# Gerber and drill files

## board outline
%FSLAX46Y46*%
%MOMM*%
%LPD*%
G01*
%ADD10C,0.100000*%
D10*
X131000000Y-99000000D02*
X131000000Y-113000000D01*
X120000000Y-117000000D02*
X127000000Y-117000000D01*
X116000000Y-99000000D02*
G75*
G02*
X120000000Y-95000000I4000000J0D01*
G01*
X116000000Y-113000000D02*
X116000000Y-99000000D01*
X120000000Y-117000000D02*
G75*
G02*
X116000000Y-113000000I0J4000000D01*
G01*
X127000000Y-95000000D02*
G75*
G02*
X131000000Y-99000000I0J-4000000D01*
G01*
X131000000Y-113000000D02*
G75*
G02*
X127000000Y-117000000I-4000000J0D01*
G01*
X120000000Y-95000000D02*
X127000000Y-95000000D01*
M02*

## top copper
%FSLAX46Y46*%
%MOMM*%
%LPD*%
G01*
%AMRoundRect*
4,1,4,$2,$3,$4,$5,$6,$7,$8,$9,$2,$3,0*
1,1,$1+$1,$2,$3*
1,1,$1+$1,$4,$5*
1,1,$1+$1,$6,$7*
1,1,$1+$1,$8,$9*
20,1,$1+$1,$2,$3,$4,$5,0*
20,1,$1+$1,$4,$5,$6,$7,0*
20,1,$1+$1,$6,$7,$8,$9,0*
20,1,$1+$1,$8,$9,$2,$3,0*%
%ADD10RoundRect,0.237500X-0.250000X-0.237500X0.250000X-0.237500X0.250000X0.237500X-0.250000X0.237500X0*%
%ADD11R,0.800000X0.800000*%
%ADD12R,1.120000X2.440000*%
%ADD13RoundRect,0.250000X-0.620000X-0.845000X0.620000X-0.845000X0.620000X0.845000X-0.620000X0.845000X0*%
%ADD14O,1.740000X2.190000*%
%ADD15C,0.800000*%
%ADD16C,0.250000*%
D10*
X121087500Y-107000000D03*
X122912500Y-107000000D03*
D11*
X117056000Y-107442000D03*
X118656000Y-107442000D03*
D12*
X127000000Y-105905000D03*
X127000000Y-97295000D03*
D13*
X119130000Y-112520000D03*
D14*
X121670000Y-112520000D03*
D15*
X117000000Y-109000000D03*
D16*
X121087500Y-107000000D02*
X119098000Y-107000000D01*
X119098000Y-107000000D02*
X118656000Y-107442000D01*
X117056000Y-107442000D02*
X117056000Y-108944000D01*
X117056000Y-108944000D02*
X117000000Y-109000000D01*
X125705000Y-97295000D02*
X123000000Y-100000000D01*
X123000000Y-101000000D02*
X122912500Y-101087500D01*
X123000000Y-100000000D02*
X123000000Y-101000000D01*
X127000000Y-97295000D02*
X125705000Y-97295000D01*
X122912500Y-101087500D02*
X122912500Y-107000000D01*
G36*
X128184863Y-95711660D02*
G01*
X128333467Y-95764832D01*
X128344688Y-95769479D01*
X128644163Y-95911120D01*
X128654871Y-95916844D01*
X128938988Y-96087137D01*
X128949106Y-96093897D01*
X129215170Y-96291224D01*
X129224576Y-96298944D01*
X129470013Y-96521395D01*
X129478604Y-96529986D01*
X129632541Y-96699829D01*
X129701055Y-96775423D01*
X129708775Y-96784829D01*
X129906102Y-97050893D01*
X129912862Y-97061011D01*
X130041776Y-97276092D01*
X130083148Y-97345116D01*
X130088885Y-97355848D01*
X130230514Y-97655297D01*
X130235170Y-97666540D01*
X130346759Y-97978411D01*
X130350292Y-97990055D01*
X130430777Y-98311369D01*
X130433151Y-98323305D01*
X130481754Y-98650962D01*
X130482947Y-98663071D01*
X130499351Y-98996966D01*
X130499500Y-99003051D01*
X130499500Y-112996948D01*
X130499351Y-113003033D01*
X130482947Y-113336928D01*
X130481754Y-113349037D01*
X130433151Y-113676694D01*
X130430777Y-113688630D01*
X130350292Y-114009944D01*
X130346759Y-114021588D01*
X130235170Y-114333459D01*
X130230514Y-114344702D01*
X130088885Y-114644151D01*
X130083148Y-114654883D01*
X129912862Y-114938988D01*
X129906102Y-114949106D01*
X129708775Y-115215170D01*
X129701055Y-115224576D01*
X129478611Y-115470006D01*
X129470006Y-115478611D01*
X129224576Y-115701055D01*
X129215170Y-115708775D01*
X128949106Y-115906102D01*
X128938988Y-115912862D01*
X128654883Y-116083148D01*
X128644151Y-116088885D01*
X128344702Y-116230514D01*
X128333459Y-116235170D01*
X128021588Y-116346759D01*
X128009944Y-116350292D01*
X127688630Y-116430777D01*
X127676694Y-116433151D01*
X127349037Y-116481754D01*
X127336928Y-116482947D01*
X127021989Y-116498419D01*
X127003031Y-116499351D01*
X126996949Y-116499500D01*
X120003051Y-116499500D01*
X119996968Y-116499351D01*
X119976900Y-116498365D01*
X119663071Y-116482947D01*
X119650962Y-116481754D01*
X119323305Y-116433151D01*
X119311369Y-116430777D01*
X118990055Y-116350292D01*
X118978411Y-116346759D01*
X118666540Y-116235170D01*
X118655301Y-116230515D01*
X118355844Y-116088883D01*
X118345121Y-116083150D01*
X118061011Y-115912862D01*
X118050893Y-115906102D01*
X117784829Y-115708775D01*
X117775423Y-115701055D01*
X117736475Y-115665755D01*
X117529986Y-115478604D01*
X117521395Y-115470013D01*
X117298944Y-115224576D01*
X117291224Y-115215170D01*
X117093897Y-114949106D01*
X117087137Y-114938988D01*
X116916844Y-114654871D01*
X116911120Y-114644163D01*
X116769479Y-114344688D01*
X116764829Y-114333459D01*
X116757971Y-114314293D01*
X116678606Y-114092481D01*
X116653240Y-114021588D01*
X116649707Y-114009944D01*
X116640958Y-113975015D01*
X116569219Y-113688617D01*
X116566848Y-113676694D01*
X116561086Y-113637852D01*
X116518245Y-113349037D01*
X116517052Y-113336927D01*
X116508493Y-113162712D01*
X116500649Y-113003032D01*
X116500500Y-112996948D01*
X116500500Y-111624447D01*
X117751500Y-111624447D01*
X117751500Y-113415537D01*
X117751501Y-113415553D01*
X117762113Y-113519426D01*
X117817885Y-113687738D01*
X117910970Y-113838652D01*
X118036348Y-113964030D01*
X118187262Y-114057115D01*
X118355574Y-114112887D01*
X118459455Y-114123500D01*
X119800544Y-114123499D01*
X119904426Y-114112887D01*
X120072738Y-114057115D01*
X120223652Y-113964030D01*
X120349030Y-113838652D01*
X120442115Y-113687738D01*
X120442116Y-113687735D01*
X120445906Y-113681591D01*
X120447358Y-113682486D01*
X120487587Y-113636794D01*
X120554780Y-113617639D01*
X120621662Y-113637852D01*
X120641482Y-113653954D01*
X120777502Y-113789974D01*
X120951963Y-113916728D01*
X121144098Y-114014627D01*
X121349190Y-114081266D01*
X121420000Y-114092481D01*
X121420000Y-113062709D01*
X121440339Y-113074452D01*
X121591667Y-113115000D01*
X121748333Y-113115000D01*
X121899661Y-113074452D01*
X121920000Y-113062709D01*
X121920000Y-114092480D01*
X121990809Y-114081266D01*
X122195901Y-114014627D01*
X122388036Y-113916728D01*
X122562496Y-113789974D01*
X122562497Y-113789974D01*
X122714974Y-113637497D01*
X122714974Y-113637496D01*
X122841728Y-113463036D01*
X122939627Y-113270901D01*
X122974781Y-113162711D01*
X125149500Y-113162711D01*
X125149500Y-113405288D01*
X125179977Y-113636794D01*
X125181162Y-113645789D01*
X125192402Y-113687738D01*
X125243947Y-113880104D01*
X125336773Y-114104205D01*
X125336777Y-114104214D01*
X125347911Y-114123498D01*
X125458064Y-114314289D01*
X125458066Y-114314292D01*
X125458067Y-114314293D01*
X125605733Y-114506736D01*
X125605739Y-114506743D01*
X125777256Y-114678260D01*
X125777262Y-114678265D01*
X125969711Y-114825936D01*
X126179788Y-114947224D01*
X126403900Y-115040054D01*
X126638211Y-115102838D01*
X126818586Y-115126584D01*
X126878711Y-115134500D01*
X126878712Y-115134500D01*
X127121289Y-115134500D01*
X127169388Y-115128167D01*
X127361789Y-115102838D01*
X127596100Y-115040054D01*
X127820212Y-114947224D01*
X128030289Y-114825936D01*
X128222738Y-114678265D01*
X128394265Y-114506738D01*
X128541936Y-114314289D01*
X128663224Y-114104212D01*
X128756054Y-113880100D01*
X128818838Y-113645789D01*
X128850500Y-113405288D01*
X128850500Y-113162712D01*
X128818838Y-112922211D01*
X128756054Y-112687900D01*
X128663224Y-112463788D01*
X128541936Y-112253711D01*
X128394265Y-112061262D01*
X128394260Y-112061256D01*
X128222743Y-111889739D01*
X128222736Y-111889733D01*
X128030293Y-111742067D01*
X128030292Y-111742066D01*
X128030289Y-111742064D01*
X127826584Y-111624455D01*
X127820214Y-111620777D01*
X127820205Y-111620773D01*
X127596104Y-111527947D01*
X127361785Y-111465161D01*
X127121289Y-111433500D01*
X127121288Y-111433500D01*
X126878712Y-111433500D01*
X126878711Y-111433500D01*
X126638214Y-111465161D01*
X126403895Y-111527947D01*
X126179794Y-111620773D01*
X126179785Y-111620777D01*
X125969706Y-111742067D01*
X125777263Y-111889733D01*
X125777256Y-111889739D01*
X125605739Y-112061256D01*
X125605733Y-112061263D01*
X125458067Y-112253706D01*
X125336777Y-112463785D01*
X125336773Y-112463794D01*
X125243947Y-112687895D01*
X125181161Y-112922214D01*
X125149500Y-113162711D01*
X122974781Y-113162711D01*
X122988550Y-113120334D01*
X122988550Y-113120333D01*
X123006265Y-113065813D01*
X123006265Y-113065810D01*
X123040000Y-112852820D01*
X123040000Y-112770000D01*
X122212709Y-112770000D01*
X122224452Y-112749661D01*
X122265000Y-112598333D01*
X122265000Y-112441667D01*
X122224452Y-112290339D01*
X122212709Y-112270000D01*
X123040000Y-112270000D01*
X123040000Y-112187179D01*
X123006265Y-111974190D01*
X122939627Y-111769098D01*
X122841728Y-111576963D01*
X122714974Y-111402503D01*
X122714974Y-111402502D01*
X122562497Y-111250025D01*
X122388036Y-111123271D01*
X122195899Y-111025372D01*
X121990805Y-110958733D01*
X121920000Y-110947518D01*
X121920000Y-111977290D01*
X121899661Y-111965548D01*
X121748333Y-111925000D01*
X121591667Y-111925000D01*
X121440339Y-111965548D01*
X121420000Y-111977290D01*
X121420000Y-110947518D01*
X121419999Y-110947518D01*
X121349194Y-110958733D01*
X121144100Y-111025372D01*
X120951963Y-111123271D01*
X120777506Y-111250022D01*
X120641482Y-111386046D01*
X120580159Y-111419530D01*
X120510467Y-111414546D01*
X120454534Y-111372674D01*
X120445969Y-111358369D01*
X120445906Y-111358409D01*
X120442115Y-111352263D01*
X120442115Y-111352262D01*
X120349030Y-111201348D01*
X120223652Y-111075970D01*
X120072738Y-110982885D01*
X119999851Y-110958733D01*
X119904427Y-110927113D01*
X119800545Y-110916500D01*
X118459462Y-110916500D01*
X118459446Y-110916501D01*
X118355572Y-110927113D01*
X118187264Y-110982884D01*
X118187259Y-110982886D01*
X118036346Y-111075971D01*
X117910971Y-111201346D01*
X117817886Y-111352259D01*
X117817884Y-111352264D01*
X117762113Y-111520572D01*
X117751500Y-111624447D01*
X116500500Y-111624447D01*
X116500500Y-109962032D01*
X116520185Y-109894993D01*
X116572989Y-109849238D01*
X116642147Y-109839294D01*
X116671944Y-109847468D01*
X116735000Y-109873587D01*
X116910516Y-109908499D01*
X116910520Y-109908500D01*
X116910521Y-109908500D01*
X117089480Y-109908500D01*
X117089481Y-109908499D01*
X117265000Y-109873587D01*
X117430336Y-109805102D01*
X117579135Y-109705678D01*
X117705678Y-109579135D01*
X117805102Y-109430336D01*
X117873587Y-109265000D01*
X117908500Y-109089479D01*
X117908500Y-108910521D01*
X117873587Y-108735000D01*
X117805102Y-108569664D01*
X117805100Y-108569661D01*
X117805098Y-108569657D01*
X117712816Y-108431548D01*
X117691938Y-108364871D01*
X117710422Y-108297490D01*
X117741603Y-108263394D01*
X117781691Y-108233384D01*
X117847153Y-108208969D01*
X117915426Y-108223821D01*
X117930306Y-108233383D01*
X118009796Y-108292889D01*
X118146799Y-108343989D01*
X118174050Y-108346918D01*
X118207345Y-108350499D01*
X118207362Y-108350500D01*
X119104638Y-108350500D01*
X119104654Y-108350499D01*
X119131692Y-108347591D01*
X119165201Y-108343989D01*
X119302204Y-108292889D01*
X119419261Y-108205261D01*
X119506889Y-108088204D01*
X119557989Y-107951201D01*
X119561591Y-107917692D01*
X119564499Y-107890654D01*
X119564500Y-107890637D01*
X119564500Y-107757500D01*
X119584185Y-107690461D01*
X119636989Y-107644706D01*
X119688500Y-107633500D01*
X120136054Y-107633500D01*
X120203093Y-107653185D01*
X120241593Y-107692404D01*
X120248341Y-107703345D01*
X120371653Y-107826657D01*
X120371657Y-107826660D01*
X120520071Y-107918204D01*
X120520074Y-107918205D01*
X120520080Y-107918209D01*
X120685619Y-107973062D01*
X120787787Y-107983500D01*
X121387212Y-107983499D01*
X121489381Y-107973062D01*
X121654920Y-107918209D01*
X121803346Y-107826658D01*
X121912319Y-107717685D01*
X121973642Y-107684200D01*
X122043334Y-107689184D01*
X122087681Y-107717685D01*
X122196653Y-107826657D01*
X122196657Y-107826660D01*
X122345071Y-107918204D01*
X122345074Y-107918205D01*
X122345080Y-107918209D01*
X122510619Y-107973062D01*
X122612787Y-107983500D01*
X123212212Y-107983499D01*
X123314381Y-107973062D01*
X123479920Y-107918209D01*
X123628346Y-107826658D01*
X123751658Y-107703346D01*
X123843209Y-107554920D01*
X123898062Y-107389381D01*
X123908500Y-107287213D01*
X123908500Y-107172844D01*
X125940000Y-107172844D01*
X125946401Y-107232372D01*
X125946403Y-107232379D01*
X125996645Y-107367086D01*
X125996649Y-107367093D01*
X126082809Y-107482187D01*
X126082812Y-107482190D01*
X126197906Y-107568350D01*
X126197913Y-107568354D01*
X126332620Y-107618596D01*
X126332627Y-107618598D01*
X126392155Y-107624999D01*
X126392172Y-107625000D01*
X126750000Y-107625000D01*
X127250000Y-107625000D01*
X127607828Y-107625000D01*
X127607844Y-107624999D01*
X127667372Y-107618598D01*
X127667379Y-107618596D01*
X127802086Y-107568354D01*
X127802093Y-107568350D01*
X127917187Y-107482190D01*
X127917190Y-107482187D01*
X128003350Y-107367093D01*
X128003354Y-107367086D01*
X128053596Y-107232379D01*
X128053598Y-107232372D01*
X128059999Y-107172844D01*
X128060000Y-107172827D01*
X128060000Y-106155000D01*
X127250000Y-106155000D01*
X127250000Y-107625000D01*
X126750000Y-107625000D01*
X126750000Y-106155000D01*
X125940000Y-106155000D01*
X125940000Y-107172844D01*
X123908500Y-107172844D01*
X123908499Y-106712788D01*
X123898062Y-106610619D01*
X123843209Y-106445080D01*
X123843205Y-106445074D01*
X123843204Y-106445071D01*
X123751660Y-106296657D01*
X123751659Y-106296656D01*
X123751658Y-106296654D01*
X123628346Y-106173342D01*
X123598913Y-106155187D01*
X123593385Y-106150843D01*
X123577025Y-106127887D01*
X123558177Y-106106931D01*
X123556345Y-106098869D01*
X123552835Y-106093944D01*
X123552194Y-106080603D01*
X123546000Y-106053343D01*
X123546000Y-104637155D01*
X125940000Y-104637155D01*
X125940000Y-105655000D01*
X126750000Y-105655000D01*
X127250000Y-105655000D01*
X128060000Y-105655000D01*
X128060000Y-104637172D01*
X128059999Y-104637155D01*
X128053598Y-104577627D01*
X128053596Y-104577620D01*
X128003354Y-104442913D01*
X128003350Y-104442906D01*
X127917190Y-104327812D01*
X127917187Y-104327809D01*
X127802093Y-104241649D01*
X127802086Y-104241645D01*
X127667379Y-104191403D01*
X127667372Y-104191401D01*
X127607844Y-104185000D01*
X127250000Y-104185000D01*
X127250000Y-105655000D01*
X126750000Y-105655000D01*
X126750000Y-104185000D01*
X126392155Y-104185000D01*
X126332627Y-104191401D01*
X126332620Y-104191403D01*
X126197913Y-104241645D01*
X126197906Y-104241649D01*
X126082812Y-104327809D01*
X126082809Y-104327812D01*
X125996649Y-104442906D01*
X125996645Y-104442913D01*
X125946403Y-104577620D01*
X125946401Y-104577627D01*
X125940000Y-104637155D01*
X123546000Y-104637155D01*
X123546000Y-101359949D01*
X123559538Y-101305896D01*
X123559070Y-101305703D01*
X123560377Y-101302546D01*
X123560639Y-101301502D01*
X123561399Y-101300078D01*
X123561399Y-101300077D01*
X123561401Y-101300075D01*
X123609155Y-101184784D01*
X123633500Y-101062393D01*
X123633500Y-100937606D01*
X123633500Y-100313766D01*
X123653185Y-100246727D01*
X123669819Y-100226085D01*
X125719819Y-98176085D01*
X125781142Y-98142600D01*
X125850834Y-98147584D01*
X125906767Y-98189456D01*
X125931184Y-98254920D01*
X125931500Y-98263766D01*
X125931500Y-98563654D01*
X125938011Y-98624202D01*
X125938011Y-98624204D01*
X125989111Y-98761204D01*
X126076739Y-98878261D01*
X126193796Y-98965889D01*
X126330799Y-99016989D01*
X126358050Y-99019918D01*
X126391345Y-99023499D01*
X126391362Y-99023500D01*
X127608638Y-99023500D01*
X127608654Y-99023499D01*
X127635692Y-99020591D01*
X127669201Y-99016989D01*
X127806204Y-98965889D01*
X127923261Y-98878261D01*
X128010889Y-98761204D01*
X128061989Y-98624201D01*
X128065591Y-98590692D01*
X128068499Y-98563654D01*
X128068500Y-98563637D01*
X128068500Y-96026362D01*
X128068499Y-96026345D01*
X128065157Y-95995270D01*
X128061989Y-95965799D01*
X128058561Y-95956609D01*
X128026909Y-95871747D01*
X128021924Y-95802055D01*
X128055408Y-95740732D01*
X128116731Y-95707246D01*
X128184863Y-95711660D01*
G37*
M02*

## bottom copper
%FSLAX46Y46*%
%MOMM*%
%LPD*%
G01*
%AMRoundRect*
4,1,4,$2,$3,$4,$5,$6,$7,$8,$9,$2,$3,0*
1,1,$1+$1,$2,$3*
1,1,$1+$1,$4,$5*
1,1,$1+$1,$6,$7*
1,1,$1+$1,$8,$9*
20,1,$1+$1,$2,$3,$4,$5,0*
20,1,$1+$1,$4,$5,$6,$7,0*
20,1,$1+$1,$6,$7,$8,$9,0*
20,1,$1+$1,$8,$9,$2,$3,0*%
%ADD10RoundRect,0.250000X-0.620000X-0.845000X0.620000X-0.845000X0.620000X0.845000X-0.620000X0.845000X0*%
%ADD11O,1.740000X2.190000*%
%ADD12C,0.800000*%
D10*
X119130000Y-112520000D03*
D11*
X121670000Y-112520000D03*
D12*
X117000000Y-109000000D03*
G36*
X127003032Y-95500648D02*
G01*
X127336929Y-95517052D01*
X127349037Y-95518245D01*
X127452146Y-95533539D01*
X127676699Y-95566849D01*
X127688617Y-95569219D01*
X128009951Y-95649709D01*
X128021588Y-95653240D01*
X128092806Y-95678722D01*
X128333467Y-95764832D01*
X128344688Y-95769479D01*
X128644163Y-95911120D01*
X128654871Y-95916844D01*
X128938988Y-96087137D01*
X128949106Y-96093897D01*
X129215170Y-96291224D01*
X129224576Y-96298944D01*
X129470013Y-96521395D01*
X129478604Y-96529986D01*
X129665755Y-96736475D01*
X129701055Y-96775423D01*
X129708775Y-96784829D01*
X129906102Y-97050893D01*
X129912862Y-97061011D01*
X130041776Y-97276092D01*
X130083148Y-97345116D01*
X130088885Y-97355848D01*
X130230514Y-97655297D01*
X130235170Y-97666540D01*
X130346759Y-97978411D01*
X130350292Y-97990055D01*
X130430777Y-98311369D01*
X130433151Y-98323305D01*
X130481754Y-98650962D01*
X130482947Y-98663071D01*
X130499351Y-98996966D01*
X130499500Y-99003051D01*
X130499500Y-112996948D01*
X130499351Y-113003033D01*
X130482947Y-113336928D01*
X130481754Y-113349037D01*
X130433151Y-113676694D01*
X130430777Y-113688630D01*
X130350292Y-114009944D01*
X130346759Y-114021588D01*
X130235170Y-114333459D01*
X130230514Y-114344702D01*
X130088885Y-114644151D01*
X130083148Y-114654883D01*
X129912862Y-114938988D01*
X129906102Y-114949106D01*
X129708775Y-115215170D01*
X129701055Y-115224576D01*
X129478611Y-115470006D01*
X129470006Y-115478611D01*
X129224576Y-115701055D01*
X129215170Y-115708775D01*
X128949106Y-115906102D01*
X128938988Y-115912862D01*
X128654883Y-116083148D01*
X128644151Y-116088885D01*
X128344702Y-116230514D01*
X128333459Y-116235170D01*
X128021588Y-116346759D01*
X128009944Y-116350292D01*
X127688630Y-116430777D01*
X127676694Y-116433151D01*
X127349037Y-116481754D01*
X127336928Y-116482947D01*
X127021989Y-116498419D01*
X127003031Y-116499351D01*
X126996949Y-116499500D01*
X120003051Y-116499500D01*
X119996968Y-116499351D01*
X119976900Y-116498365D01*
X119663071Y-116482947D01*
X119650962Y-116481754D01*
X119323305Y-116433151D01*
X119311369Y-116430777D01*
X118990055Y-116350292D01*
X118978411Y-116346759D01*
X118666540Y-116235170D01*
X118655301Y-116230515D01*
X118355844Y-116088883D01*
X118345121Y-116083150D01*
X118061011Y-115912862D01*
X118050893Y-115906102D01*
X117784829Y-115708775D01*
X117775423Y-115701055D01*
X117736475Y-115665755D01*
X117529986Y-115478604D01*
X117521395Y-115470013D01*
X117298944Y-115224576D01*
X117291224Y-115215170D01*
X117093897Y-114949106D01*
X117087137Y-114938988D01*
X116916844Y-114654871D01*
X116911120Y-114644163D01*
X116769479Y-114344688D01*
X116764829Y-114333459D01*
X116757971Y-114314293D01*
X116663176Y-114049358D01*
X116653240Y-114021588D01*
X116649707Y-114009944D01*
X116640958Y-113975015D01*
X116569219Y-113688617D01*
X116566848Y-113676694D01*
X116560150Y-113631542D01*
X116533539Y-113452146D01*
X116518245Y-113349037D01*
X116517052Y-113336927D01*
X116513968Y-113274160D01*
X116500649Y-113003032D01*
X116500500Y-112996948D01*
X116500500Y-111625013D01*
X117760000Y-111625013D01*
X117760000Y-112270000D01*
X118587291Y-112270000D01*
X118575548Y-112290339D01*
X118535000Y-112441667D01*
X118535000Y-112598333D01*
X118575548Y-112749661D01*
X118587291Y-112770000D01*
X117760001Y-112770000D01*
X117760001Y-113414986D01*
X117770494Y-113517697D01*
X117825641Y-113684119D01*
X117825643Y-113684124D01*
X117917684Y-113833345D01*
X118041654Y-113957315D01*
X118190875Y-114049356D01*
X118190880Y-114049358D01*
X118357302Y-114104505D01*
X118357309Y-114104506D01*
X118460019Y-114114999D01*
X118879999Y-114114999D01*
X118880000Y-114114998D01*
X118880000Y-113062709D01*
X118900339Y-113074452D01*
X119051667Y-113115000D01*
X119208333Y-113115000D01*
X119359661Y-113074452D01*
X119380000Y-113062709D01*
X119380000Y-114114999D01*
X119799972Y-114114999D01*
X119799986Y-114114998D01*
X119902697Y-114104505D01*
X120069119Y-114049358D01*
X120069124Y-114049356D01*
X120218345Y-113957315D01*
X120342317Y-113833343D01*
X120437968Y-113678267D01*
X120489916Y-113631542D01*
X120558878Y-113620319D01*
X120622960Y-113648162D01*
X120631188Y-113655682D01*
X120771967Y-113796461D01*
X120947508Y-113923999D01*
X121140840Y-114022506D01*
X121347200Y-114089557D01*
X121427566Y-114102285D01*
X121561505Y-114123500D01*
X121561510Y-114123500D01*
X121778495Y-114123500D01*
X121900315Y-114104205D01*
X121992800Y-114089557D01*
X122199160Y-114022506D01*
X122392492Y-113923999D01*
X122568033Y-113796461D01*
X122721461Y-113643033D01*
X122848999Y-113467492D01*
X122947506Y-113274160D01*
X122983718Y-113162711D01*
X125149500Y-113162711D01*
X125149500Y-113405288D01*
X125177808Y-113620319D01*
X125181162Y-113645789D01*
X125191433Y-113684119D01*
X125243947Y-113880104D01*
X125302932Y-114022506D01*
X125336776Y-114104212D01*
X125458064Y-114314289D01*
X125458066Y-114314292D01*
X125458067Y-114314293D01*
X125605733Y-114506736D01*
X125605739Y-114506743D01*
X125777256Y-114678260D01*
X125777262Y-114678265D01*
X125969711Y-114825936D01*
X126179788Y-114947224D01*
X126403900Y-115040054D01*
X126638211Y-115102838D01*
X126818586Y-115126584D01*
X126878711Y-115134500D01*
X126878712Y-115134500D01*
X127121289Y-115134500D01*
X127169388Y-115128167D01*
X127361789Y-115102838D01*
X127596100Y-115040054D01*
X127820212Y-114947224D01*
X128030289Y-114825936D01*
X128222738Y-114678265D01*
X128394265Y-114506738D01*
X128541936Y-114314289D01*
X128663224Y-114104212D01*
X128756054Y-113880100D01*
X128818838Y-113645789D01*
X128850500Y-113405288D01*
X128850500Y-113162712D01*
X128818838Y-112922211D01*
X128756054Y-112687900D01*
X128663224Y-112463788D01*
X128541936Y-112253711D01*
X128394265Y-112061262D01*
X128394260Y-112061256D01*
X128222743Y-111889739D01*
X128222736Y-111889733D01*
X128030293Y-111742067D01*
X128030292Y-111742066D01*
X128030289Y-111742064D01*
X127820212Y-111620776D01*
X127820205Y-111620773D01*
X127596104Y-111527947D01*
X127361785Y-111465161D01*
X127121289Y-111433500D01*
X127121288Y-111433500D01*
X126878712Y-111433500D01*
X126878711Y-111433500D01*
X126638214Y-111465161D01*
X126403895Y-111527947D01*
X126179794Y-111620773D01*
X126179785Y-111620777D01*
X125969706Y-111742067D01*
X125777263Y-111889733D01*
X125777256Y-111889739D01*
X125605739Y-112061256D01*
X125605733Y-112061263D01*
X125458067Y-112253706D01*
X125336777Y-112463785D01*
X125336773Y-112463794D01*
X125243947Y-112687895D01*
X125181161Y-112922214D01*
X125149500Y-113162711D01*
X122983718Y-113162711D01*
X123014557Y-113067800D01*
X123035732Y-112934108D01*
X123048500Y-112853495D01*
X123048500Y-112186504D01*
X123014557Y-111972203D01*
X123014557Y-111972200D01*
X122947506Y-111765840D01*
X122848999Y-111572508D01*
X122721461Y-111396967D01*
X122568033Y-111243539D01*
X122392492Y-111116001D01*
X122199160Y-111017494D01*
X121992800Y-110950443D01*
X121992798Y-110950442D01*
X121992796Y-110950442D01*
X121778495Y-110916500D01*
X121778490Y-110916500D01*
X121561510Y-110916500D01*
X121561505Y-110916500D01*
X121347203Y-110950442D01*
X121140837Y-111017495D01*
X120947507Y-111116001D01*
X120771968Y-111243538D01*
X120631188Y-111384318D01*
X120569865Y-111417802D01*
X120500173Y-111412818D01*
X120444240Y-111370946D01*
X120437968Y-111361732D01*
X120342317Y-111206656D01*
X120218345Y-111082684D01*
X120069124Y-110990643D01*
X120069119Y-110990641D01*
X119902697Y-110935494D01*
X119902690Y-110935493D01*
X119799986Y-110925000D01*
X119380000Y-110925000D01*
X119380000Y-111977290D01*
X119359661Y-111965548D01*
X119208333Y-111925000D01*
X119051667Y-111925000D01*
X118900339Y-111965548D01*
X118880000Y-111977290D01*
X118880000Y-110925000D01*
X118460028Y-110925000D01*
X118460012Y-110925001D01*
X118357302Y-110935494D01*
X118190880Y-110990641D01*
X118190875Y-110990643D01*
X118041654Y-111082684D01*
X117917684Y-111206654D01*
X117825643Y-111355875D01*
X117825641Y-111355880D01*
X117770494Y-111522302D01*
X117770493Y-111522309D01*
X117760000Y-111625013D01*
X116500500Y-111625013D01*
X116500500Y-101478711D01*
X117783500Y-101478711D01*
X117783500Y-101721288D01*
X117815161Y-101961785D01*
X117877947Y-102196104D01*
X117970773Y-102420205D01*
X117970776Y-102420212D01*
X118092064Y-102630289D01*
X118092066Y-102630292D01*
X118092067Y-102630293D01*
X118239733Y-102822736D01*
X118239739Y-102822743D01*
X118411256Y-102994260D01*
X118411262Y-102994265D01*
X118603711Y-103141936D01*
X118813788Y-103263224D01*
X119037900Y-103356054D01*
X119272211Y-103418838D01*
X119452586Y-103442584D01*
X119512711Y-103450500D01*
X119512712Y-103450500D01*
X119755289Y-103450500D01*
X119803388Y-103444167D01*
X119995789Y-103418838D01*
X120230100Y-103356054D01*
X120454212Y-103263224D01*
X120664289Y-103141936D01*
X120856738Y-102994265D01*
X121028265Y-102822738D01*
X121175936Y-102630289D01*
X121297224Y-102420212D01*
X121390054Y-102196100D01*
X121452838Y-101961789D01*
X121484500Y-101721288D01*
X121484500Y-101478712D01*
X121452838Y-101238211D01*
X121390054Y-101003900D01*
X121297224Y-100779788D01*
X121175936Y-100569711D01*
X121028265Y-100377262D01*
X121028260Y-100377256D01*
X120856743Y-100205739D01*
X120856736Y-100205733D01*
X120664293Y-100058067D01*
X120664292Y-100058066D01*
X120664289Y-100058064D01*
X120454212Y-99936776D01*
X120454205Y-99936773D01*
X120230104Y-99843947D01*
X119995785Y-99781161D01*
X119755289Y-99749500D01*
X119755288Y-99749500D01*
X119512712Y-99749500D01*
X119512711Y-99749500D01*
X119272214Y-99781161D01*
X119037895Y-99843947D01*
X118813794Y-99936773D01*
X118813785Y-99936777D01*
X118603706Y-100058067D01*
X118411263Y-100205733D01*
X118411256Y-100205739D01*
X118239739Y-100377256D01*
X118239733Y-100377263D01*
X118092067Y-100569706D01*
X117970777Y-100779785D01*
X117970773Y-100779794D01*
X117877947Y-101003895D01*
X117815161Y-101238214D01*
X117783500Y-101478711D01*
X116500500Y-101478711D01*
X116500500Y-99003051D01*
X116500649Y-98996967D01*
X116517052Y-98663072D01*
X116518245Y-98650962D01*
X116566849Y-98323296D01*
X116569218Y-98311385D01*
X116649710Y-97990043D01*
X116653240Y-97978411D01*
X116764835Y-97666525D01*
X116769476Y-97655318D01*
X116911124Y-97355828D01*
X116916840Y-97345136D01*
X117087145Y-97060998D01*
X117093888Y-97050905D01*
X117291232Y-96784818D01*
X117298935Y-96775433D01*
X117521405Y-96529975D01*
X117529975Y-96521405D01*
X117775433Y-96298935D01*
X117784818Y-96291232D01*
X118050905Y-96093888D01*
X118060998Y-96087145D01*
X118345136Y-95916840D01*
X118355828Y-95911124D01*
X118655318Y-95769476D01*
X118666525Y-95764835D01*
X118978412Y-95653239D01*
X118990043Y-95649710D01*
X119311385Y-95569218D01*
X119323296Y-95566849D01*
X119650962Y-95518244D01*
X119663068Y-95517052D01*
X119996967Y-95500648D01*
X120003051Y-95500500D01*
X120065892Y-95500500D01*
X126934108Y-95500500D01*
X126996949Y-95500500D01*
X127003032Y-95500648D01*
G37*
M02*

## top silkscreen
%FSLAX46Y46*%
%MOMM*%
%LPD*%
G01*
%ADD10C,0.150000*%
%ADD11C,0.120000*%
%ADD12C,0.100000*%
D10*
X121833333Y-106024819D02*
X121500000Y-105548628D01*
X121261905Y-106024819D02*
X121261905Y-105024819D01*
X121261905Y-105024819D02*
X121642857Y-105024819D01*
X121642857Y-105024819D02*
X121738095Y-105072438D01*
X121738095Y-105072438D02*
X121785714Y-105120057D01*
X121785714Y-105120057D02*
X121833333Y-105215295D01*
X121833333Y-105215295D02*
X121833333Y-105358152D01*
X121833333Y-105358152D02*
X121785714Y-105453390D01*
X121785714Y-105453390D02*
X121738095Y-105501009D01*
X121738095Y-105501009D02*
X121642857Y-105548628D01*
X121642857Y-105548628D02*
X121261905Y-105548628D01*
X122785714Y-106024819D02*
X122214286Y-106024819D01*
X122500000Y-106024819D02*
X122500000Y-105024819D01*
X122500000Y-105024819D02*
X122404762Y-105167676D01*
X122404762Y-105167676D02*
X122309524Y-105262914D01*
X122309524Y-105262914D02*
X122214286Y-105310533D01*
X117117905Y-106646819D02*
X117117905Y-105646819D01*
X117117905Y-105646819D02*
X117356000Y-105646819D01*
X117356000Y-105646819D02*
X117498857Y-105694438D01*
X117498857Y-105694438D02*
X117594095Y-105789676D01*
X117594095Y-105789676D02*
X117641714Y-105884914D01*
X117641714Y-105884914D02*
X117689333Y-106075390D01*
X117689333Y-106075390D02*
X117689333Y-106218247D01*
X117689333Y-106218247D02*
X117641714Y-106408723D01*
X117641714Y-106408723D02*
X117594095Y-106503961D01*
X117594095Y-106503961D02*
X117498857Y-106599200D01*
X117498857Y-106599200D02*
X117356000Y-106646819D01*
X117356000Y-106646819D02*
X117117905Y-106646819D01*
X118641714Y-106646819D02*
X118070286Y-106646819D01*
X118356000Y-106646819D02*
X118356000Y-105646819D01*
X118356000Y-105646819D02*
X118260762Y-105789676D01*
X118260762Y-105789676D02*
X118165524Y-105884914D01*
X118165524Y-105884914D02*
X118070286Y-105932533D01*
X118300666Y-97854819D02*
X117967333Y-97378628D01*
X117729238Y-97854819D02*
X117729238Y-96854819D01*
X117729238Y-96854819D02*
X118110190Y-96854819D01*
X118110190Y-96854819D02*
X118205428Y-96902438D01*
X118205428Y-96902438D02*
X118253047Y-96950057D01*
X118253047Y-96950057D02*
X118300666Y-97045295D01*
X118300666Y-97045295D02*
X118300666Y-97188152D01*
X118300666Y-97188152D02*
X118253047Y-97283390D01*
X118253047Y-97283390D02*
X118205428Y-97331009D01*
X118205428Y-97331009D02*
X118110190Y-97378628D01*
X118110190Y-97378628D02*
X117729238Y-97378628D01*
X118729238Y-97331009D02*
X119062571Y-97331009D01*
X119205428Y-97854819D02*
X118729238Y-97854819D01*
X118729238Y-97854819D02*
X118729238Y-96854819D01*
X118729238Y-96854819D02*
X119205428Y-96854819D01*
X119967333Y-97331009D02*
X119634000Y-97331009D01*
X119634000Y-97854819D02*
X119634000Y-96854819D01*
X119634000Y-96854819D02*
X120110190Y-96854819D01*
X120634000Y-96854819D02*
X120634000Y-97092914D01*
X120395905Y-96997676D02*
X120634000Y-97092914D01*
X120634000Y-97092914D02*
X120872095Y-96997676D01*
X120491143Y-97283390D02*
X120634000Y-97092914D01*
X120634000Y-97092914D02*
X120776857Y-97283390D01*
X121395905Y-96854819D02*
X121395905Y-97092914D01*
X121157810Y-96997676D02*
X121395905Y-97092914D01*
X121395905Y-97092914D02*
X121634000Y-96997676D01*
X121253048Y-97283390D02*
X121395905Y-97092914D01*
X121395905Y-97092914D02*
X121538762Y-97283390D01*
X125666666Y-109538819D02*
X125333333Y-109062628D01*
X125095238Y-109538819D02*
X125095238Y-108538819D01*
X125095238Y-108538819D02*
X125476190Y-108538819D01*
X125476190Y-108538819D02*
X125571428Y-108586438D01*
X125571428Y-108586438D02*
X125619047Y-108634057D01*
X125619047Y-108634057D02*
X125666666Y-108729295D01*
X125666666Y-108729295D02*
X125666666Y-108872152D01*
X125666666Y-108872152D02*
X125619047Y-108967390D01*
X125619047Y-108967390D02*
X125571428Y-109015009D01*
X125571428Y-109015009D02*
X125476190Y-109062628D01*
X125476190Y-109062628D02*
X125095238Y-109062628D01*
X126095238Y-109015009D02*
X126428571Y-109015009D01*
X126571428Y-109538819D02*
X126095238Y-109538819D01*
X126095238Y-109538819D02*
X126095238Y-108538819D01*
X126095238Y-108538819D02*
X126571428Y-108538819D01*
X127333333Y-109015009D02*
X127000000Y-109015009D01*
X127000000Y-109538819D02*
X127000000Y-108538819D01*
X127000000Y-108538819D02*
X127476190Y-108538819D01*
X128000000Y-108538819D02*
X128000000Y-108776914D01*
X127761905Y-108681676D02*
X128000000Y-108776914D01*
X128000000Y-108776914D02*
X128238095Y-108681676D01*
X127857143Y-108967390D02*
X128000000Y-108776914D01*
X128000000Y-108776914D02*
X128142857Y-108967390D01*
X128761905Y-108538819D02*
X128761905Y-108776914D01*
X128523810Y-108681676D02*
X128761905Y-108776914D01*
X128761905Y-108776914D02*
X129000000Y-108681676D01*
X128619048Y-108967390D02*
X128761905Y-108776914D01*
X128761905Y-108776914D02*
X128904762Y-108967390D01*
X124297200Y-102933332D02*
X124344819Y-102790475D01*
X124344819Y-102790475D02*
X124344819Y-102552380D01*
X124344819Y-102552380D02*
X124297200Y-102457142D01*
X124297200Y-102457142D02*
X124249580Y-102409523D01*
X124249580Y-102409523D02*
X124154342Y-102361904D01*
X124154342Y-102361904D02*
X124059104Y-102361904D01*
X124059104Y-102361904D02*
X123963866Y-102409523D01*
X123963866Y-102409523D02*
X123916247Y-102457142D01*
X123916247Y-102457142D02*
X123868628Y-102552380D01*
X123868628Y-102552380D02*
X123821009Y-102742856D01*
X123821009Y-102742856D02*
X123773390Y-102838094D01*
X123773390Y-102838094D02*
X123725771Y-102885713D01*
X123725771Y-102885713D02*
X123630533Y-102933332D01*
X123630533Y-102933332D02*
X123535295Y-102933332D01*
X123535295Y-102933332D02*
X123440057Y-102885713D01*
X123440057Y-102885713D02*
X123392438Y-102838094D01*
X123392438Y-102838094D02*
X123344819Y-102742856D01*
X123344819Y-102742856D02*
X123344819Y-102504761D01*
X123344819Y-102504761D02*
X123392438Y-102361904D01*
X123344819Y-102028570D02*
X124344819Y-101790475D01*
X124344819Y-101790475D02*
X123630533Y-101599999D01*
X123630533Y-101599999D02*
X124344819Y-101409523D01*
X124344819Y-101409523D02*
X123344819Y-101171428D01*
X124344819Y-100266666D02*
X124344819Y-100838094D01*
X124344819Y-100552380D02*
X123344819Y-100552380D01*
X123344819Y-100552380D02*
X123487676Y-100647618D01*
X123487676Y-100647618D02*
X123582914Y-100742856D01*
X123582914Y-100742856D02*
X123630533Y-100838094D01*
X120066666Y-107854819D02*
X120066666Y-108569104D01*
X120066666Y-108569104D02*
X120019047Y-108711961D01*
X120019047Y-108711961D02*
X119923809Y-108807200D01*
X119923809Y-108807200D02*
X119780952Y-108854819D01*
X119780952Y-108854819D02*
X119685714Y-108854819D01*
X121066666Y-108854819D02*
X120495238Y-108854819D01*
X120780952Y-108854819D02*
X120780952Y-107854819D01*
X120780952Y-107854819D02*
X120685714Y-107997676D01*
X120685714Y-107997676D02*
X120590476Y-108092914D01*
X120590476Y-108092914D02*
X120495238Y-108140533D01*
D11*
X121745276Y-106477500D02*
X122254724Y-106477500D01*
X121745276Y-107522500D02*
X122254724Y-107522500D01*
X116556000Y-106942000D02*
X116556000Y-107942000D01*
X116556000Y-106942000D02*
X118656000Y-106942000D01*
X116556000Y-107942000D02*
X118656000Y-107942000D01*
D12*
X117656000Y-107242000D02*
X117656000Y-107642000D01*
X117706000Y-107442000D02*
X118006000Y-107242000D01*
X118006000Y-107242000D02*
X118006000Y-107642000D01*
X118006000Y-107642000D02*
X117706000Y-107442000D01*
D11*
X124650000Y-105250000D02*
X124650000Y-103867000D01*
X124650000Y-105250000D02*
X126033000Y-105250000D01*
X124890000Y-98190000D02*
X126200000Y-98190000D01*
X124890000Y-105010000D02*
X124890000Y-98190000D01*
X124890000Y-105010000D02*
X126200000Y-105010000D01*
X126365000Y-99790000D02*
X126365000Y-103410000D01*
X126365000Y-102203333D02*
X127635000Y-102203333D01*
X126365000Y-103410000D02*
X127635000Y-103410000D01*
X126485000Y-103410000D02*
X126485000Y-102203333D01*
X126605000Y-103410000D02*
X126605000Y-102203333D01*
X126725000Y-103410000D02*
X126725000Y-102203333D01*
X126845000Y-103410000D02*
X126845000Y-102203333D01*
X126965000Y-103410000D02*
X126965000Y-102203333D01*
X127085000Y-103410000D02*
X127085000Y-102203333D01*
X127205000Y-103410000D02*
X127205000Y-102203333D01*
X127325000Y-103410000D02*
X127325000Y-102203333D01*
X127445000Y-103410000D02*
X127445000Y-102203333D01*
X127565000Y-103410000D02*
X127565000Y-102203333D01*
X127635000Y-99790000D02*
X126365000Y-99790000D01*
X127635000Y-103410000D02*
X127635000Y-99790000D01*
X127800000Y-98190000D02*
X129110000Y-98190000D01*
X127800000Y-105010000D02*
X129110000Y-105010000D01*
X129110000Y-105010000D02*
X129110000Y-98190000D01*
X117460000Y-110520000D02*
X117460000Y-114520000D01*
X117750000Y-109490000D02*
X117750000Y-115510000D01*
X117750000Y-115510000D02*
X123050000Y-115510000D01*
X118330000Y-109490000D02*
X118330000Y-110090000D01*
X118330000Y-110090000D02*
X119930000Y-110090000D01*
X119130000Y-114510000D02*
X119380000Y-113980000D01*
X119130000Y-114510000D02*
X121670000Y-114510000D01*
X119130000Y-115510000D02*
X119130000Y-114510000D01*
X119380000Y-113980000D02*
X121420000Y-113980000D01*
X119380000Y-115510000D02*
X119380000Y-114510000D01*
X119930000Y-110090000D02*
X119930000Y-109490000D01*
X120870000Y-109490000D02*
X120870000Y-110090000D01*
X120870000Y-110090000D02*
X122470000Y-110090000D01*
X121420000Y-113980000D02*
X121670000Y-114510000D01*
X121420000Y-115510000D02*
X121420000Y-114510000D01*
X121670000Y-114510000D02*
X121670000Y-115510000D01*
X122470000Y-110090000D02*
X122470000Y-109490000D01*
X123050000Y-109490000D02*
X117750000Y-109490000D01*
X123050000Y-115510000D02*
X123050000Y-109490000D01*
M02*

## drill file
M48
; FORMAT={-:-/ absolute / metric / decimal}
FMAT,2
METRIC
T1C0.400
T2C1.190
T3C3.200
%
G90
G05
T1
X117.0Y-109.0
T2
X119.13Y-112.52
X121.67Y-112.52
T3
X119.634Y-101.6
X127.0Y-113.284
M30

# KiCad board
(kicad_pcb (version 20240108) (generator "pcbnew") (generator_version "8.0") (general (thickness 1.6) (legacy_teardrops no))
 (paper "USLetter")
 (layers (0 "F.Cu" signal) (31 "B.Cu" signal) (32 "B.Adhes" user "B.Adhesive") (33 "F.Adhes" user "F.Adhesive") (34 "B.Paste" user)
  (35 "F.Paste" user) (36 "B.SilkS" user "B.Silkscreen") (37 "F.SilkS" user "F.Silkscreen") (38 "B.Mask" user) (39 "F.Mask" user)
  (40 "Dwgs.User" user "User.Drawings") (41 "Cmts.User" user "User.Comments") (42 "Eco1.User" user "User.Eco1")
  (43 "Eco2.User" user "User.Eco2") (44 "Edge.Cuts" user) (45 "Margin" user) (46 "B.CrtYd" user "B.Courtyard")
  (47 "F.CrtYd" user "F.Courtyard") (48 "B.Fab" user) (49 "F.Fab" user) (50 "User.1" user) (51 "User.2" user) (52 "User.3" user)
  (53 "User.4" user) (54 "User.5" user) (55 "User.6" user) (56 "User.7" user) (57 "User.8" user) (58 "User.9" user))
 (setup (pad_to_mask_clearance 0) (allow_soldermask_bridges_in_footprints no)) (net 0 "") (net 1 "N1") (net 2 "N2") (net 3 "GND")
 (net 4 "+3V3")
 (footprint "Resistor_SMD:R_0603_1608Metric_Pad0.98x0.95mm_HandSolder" (layer "F.Cu") (at 122 107)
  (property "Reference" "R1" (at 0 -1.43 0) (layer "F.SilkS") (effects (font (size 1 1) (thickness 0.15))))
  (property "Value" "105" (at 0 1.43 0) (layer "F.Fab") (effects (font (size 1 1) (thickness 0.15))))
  (fp_line (start -0.254724 -0.5225) (end 0.254724 -0.5225) (stroke (width 0.12) (type solid)) (layer "F.SilkS"))
  (fp_line (start -0.254724 0.5225) (end 0.254724 0.5225) (stroke (width 0.12) (type solid)) (layer "F.SilkS"))
  (pad "1" smd roundrect (at -0.9125 0) (size 0.975 0.95) (layers "F.Cu" "F.Paste" "F.Mask") (roundrect_rratio 0.25) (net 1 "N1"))
  (pad "2" smd roundrect (at 0.9125 0) (size 0.975 0.95) (layers "F.Cu" "F.Paste" "F.Mask") (roundrect_rratio 0.25) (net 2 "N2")))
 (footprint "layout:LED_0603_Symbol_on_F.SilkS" (layer "F.Cu") (at 117.856 107.442)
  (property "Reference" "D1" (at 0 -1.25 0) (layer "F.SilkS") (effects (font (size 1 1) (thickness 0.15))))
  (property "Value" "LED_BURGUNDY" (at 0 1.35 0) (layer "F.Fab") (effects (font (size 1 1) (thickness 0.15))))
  (fp_line (start -1.3 -0.5) (end -1.3 0.5) (stroke (width 0.12) (type solid)) (layer "F.SilkS"))
  (fp_line (start -1.3 -0.5) (end 0.8 -0.5) (stroke (width 0.12) (type solid)) (layer "F.SilkS"))
  (fp_line (start -1.3 0.5) (end 0.8 0.5) (stroke (width 0.12) (type solid)) (layer "F.SilkS"))
  (fp_line (start -0.2 -0.2) (end -0.2 0.2) (stroke (width 0.1) (type solid)) (layer "F.SilkS"))
  (fp_line (start -0.15 0) (end 0.15 -0.2) (stroke (width 0.1) (type solid)) (layer "F.SilkS"))
  (fp_line (start 0.15 -0.2) (end 0.15 0.2) (stroke (width 0.1) (type solid)) (layer "F.SilkS"))
  (fp_line (start 0.15 0.2) (end -0.15 0) (stroke (width 0.1) (type solid)) (layer "F.SilkS"))
  (pad "1" smd rect (at -0.8 0 180) (size 0.8 0.8) (layers "F.Cu" "F.Paste" "F.Mask") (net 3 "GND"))
  (pad "2" smd rect (at 0.8 0 180) (size 0.8 0.8) (layers "F.Cu" "F.Paste" "F.Mask") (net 1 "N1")))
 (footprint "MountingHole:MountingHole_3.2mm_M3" (layer "F.Cu") (at 119.634 101.6)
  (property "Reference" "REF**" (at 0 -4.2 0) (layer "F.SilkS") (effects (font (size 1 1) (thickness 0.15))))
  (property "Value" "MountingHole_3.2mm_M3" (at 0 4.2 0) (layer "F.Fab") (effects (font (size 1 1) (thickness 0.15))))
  (pad "" np_thru_hole circle (at 0 0) (size 3.2 3.2) (drill 3.2) (layers "F&B.Cu" "*.Mask")))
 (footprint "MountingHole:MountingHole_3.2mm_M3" (layer "F.Cu") (at 127 113.284)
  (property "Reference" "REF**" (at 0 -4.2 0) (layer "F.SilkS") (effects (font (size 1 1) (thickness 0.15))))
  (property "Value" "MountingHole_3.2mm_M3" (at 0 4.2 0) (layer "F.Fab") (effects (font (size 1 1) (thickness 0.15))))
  (pad "" np_thru_hole circle (at 0 0) (size 3.2 3.2) (drill 3.2) (layers "*.Cu" "*.Mask")))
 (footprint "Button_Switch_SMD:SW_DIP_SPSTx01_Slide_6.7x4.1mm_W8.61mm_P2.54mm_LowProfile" (layer "F.Cu") (at 127 101.6 90)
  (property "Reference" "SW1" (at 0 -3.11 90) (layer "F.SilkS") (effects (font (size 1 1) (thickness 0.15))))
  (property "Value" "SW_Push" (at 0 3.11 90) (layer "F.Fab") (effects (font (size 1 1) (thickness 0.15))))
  (fp_line (start -3.65 -2.35) (end -2.267 -2.35) (stroke (width 0.12) (type solid)) (layer "F.SilkS"))
  (fp_line (start -3.65 -2.35) (end -3.65 -0.967) (stroke (width 0.12) (type solid)) (layer "F.SilkS"))
  (fp_line (start 3.41 -2.11) (end 3.41 -0.8) (stroke (width 0.12) (type solid)) (layer "F.SilkS"))
  (fp_line (start -3.41 -2.11) (end 3.41 -2.11) (stroke (width 0.12) (type solid)) (layer "F.SilkS"))
  (fp_line (start -3.41 -2.11) (end -3.41 -0.8) (stroke (width 0.12) (type solid)) (layer "F.SilkS"))
  (fp_line (start 1.81 -0.635) (end -1.81 -0.635) (stroke (width 0.12) (type solid)) (layer "F.SilkS"))
  (fp_line (start -0.603333 -0.635) (end -0.603333 0.635) (stroke (width 0.12) (type solid)) (layer "F.SilkS"))
  (fp_line (start -1.81 -0.635) (end -1.81 0.635) (stroke (width 0.12) (type solid)) (layer "F.SilkS"))
  (fp_line (start -1.81 -0.515) (end -0.603333 -0.515) (stroke (width 0.12) (type solid)) (layer "F.SilkS"))
  (fp_line (start -1.81 -0.395) (end -0.603333 -0.395) (stroke (width 0.12) (type solid)) (layer "F.SilkS"))
  (fp_line (start -1.81 -0.275) (end -0.603333 -0.275) (stroke (width 0.12) (type solid)) (layer "F.SilkS"))
  (fp_line (start -1.81 -0.155) (end -0.603333 -0.155) (stroke (width 0.12) (type solid)) (layer "F.SilkS"))
  (fp_line (start -1.81 -0.035) (end -0.603333 -0.035) (stroke (width 0.12) (type solid)) (layer "F.SilkS"))
  (fp_line (start -1.81 0.085) (end -0.603333 0.085) (stroke (width 0.12) (type solid)) (layer "F.SilkS"))
  (fp_line (start -1.81 0.205) (end -0.603333 0.205) (stroke (width 0.12) (type solid)) (layer "F.SilkS"))
  (fp_line (start -1.81 0.325) (end -0.603333 0.325) (stroke (width 0.12) (type solid)) (layer "F.SilkS"))
  (fp_line (start -1.81 0.445) (end -0.603333 0.445) (stroke (width 0.12) (type solid)) (layer "F.SilkS"))
  (fp_line (start -1.81 0.565) (end -0.603333 0.565) (stroke (width 0.12) (type solid)) (layer "F.SilkS"))
  (fp_line (start 1.81 0.635) (end 1.81 -0.635) (stroke (width 0.12) (type solid)) (layer "F.SilkS"))
  (fp_line (start -1.81 0.635) (end 1.81 0.635) (stroke (width 0.12) (type solid)) (layer "F.SilkS"))
  (fp_line (start 3.41 0.8) (end 3.41 2.11) (stroke (width 0.12) (type solid)) (layer "F.SilkS"))
  (fp_line (start -3.41 0.8) (end -3.41 2.11) (stroke (width 0.12) (type solid)) (layer "F.SilkS"))
  (fp_line (start -3.41 2.11) (end 3.41 2.11) (stroke (width 0.12) (type solid)) (layer "F.SilkS"))
  (pad "1" smd rect (at -4.305 0 90) (size 2.44 1.12) (layers "F.Cu" "F.Paste" "F.Mask") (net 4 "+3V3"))
  (pad "2" smd rect (at 4.305 0 90) (size 2.44 1.12) (layers "F.Cu" "F.Paste" "F.Mask") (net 2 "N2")))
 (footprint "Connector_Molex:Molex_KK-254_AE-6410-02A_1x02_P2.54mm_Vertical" (layer "F.Cu") (at 119.13 112.52)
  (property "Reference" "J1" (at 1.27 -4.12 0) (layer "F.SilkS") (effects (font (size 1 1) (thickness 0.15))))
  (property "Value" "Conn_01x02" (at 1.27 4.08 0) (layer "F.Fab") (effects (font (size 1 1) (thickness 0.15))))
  (fp_line (start -1.67 -2) (end -1.67 2) (stroke (width 0.12) (type solid)) (layer "F.SilkS"))
  (fp_line (start -1.38 -3.03) (end -1.38 2.99) (stroke (width 0.12) (type solid)) (layer "F.SilkS"))
  (fp_line (start -1.38 2.99) (end 3.92 2.99) (stroke (width 0.12) (type solid)) (layer "F.SilkS"))
  (fp_line (start -0.8 -3.03) (end -0.8 -2.43) (stroke (width 0.12) (type solid)) (layer "F.SilkS"))
  (fp_line (start -0.8 -2.43) (end 0.8 -2.43) (stroke (width 0.12) (type solid)) (layer "F.SilkS"))
  (fp_line (start 0 1.99) (end 0.25 1.46) (stroke (width 0.12) (type solid)) (layer "F.SilkS"))
  (fp_line (start 0 1.99) (end 2.54 1.99) (stroke (width 0.12) (type solid)) (layer "F.SilkS"))
  (fp_line (start 0 2.99) (end 0 1.99) (stroke (width 0.12) (type solid)) (layer "F.SilkS"))
  (fp_line (start 0.25 1.46) (end 2.29 1.46) (stroke (width 0.12) (type solid)) (layer "F.SilkS"))
  (fp_line (start 0.25 2.99) (end 0.25 1.99) (stroke (width 0.12) (type solid)) (layer "F.SilkS"))
  (fp_line (start 0.8 -2.43) (end 0.8 -3.03) (stroke (width 0.12) (type solid)) (layer "F.SilkS"))
  (fp_line (start 1.74 -3.03) (end 1.74 -2.43) (stroke (width 0.12) (type solid)) (layer "F.SilkS"))
  (fp_line (start 1.74 -2.43) (end 3.34 -2.43) (stroke (width 0.12) (type solid)) (layer "F.SilkS"))
  (fp_line (start 2.29 1.46) (end 2.54 1.99) (stroke (width 0.12) (type solid)) (layer "F.SilkS"))
  (fp_line (start 2.29 2.99) (end 2.29 1.99) (stroke (width 0.12) (type solid)) (layer "F.SilkS"))
  (fp_line (start 2.54 1.99) (end 2.54 2.99) (stroke (width 0.12) (type solid)) (layer "F.SilkS"))
  (fp_line (start 3.34 -2.43) (end 3.34 -3.03) (stroke (width 0.12) (type solid)) (layer "F.SilkS"))
  (fp_line (start 3.92 -3.03) (end -1.38 -3.03) (stroke (width 0.12) (type solid)) (layer "F.SilkS"))
  (fp_line (start 3.92 2.99) (end 3.92 -3.03) (stroke (width 0.12) (type solid)) (layer "F.SilkS"))
  (pad "1" thru_hole roundrect (at 0 0) (size 1.74 2.19) (drill 1.19) (layers "*.Cu" "*.Mask") (remove_unused_layers no)
   (roundrect_rratio 0.143678) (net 3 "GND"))
  (pad "2" thru_hole oval (at 2.54 0) (size 1.74 2.19) (drill 1.19) (layers "*.Cu" "*.Mask") (remove_unused_layers no) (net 4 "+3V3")))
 (gr_line (start 131 99) (end 131 113) (stroke (width 0.1) (type default)) (layer "Edge.Cuts"))
 (gr_line (start 120 117) (end 127 117) (stroke (width 0.1) (type default)) (layer "Edge.Cuts"))
 (gr_arc (start 116 99) (mid 117.171573 96.171573) (end 120 95) (stroke (width 0.1) (type default)) (layer "Edge.Cuts"))
 (gr_line (start 116 113) (end 116 99) (stroke (width 0.1) (type default)) (layer "Edge.Cuts"))
 (gr_arc (start 120 117) (mid 117.171573 115.828427) (end 116 113) (stroke (width 0.1) (type default)) (layer "Edge.Cuts"))
 (gr_arc (start 127 95) (mid 129.828427 96.171573) (end 131 99) (stroke (width 0.1) (type default)) (layer "Edge.Cuts"))
 (gr_arc (start 131 113) (mid 129.828427 115.828427) (end 127 117) (stroke (width 0.1) (type default)) (layer "Edge.Cuts"))
 (gr_line (start 120 95) (end 127 95) (stroke (width 0.1) (type default)) (layer "Edge.Cuts"))
 (segment (start 121.0875 107) (end 119.098 107) (width 0.25) (layer "F.Cu") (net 1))
 (segment (start 119.098 107) (end 118.656 107.442) (width 0.25) (layer "F.Cu") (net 1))
 (segment (start 117.056 107.442) (end 117.056 108.944) (width 0.25) (layer "F.Cu") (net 3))
 (segment (start 117.056 108.944) (end 117 109) (width 0.25) (layer "F.Cu") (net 3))
 (via (at 117 109) (size 0.8) (drill 0.4) (layers "F.Cu" "B.Cu") (free yes) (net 3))
 (segment (start 125.705 97.295) (end 123 100) (width 0.25) (layer "F.Cu") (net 2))
 (segment (start 123 101) (end 122.9125 101.0875) (width 0.25) (layer "F.Cu") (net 2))
 (segment (start 123 100) (end 123 101) (width 0.25) (layer "F.Cu") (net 2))
 (segment (start 127 97.295) (end 125.705 97.295) (width 0.25) (layer "F.Cu") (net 2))
 (segment (start 122.9125 101.0875) (end 122.9125 107) (width 0.25) (layer "F.Cu") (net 2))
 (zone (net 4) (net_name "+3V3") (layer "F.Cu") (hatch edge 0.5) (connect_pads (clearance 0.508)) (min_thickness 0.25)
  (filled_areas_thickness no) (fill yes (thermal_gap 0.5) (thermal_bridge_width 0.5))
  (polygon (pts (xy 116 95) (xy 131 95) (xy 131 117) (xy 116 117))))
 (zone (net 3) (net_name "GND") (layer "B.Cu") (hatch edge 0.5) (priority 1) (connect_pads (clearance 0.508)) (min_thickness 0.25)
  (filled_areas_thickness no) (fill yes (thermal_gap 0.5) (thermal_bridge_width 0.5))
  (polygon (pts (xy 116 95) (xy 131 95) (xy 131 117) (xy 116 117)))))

